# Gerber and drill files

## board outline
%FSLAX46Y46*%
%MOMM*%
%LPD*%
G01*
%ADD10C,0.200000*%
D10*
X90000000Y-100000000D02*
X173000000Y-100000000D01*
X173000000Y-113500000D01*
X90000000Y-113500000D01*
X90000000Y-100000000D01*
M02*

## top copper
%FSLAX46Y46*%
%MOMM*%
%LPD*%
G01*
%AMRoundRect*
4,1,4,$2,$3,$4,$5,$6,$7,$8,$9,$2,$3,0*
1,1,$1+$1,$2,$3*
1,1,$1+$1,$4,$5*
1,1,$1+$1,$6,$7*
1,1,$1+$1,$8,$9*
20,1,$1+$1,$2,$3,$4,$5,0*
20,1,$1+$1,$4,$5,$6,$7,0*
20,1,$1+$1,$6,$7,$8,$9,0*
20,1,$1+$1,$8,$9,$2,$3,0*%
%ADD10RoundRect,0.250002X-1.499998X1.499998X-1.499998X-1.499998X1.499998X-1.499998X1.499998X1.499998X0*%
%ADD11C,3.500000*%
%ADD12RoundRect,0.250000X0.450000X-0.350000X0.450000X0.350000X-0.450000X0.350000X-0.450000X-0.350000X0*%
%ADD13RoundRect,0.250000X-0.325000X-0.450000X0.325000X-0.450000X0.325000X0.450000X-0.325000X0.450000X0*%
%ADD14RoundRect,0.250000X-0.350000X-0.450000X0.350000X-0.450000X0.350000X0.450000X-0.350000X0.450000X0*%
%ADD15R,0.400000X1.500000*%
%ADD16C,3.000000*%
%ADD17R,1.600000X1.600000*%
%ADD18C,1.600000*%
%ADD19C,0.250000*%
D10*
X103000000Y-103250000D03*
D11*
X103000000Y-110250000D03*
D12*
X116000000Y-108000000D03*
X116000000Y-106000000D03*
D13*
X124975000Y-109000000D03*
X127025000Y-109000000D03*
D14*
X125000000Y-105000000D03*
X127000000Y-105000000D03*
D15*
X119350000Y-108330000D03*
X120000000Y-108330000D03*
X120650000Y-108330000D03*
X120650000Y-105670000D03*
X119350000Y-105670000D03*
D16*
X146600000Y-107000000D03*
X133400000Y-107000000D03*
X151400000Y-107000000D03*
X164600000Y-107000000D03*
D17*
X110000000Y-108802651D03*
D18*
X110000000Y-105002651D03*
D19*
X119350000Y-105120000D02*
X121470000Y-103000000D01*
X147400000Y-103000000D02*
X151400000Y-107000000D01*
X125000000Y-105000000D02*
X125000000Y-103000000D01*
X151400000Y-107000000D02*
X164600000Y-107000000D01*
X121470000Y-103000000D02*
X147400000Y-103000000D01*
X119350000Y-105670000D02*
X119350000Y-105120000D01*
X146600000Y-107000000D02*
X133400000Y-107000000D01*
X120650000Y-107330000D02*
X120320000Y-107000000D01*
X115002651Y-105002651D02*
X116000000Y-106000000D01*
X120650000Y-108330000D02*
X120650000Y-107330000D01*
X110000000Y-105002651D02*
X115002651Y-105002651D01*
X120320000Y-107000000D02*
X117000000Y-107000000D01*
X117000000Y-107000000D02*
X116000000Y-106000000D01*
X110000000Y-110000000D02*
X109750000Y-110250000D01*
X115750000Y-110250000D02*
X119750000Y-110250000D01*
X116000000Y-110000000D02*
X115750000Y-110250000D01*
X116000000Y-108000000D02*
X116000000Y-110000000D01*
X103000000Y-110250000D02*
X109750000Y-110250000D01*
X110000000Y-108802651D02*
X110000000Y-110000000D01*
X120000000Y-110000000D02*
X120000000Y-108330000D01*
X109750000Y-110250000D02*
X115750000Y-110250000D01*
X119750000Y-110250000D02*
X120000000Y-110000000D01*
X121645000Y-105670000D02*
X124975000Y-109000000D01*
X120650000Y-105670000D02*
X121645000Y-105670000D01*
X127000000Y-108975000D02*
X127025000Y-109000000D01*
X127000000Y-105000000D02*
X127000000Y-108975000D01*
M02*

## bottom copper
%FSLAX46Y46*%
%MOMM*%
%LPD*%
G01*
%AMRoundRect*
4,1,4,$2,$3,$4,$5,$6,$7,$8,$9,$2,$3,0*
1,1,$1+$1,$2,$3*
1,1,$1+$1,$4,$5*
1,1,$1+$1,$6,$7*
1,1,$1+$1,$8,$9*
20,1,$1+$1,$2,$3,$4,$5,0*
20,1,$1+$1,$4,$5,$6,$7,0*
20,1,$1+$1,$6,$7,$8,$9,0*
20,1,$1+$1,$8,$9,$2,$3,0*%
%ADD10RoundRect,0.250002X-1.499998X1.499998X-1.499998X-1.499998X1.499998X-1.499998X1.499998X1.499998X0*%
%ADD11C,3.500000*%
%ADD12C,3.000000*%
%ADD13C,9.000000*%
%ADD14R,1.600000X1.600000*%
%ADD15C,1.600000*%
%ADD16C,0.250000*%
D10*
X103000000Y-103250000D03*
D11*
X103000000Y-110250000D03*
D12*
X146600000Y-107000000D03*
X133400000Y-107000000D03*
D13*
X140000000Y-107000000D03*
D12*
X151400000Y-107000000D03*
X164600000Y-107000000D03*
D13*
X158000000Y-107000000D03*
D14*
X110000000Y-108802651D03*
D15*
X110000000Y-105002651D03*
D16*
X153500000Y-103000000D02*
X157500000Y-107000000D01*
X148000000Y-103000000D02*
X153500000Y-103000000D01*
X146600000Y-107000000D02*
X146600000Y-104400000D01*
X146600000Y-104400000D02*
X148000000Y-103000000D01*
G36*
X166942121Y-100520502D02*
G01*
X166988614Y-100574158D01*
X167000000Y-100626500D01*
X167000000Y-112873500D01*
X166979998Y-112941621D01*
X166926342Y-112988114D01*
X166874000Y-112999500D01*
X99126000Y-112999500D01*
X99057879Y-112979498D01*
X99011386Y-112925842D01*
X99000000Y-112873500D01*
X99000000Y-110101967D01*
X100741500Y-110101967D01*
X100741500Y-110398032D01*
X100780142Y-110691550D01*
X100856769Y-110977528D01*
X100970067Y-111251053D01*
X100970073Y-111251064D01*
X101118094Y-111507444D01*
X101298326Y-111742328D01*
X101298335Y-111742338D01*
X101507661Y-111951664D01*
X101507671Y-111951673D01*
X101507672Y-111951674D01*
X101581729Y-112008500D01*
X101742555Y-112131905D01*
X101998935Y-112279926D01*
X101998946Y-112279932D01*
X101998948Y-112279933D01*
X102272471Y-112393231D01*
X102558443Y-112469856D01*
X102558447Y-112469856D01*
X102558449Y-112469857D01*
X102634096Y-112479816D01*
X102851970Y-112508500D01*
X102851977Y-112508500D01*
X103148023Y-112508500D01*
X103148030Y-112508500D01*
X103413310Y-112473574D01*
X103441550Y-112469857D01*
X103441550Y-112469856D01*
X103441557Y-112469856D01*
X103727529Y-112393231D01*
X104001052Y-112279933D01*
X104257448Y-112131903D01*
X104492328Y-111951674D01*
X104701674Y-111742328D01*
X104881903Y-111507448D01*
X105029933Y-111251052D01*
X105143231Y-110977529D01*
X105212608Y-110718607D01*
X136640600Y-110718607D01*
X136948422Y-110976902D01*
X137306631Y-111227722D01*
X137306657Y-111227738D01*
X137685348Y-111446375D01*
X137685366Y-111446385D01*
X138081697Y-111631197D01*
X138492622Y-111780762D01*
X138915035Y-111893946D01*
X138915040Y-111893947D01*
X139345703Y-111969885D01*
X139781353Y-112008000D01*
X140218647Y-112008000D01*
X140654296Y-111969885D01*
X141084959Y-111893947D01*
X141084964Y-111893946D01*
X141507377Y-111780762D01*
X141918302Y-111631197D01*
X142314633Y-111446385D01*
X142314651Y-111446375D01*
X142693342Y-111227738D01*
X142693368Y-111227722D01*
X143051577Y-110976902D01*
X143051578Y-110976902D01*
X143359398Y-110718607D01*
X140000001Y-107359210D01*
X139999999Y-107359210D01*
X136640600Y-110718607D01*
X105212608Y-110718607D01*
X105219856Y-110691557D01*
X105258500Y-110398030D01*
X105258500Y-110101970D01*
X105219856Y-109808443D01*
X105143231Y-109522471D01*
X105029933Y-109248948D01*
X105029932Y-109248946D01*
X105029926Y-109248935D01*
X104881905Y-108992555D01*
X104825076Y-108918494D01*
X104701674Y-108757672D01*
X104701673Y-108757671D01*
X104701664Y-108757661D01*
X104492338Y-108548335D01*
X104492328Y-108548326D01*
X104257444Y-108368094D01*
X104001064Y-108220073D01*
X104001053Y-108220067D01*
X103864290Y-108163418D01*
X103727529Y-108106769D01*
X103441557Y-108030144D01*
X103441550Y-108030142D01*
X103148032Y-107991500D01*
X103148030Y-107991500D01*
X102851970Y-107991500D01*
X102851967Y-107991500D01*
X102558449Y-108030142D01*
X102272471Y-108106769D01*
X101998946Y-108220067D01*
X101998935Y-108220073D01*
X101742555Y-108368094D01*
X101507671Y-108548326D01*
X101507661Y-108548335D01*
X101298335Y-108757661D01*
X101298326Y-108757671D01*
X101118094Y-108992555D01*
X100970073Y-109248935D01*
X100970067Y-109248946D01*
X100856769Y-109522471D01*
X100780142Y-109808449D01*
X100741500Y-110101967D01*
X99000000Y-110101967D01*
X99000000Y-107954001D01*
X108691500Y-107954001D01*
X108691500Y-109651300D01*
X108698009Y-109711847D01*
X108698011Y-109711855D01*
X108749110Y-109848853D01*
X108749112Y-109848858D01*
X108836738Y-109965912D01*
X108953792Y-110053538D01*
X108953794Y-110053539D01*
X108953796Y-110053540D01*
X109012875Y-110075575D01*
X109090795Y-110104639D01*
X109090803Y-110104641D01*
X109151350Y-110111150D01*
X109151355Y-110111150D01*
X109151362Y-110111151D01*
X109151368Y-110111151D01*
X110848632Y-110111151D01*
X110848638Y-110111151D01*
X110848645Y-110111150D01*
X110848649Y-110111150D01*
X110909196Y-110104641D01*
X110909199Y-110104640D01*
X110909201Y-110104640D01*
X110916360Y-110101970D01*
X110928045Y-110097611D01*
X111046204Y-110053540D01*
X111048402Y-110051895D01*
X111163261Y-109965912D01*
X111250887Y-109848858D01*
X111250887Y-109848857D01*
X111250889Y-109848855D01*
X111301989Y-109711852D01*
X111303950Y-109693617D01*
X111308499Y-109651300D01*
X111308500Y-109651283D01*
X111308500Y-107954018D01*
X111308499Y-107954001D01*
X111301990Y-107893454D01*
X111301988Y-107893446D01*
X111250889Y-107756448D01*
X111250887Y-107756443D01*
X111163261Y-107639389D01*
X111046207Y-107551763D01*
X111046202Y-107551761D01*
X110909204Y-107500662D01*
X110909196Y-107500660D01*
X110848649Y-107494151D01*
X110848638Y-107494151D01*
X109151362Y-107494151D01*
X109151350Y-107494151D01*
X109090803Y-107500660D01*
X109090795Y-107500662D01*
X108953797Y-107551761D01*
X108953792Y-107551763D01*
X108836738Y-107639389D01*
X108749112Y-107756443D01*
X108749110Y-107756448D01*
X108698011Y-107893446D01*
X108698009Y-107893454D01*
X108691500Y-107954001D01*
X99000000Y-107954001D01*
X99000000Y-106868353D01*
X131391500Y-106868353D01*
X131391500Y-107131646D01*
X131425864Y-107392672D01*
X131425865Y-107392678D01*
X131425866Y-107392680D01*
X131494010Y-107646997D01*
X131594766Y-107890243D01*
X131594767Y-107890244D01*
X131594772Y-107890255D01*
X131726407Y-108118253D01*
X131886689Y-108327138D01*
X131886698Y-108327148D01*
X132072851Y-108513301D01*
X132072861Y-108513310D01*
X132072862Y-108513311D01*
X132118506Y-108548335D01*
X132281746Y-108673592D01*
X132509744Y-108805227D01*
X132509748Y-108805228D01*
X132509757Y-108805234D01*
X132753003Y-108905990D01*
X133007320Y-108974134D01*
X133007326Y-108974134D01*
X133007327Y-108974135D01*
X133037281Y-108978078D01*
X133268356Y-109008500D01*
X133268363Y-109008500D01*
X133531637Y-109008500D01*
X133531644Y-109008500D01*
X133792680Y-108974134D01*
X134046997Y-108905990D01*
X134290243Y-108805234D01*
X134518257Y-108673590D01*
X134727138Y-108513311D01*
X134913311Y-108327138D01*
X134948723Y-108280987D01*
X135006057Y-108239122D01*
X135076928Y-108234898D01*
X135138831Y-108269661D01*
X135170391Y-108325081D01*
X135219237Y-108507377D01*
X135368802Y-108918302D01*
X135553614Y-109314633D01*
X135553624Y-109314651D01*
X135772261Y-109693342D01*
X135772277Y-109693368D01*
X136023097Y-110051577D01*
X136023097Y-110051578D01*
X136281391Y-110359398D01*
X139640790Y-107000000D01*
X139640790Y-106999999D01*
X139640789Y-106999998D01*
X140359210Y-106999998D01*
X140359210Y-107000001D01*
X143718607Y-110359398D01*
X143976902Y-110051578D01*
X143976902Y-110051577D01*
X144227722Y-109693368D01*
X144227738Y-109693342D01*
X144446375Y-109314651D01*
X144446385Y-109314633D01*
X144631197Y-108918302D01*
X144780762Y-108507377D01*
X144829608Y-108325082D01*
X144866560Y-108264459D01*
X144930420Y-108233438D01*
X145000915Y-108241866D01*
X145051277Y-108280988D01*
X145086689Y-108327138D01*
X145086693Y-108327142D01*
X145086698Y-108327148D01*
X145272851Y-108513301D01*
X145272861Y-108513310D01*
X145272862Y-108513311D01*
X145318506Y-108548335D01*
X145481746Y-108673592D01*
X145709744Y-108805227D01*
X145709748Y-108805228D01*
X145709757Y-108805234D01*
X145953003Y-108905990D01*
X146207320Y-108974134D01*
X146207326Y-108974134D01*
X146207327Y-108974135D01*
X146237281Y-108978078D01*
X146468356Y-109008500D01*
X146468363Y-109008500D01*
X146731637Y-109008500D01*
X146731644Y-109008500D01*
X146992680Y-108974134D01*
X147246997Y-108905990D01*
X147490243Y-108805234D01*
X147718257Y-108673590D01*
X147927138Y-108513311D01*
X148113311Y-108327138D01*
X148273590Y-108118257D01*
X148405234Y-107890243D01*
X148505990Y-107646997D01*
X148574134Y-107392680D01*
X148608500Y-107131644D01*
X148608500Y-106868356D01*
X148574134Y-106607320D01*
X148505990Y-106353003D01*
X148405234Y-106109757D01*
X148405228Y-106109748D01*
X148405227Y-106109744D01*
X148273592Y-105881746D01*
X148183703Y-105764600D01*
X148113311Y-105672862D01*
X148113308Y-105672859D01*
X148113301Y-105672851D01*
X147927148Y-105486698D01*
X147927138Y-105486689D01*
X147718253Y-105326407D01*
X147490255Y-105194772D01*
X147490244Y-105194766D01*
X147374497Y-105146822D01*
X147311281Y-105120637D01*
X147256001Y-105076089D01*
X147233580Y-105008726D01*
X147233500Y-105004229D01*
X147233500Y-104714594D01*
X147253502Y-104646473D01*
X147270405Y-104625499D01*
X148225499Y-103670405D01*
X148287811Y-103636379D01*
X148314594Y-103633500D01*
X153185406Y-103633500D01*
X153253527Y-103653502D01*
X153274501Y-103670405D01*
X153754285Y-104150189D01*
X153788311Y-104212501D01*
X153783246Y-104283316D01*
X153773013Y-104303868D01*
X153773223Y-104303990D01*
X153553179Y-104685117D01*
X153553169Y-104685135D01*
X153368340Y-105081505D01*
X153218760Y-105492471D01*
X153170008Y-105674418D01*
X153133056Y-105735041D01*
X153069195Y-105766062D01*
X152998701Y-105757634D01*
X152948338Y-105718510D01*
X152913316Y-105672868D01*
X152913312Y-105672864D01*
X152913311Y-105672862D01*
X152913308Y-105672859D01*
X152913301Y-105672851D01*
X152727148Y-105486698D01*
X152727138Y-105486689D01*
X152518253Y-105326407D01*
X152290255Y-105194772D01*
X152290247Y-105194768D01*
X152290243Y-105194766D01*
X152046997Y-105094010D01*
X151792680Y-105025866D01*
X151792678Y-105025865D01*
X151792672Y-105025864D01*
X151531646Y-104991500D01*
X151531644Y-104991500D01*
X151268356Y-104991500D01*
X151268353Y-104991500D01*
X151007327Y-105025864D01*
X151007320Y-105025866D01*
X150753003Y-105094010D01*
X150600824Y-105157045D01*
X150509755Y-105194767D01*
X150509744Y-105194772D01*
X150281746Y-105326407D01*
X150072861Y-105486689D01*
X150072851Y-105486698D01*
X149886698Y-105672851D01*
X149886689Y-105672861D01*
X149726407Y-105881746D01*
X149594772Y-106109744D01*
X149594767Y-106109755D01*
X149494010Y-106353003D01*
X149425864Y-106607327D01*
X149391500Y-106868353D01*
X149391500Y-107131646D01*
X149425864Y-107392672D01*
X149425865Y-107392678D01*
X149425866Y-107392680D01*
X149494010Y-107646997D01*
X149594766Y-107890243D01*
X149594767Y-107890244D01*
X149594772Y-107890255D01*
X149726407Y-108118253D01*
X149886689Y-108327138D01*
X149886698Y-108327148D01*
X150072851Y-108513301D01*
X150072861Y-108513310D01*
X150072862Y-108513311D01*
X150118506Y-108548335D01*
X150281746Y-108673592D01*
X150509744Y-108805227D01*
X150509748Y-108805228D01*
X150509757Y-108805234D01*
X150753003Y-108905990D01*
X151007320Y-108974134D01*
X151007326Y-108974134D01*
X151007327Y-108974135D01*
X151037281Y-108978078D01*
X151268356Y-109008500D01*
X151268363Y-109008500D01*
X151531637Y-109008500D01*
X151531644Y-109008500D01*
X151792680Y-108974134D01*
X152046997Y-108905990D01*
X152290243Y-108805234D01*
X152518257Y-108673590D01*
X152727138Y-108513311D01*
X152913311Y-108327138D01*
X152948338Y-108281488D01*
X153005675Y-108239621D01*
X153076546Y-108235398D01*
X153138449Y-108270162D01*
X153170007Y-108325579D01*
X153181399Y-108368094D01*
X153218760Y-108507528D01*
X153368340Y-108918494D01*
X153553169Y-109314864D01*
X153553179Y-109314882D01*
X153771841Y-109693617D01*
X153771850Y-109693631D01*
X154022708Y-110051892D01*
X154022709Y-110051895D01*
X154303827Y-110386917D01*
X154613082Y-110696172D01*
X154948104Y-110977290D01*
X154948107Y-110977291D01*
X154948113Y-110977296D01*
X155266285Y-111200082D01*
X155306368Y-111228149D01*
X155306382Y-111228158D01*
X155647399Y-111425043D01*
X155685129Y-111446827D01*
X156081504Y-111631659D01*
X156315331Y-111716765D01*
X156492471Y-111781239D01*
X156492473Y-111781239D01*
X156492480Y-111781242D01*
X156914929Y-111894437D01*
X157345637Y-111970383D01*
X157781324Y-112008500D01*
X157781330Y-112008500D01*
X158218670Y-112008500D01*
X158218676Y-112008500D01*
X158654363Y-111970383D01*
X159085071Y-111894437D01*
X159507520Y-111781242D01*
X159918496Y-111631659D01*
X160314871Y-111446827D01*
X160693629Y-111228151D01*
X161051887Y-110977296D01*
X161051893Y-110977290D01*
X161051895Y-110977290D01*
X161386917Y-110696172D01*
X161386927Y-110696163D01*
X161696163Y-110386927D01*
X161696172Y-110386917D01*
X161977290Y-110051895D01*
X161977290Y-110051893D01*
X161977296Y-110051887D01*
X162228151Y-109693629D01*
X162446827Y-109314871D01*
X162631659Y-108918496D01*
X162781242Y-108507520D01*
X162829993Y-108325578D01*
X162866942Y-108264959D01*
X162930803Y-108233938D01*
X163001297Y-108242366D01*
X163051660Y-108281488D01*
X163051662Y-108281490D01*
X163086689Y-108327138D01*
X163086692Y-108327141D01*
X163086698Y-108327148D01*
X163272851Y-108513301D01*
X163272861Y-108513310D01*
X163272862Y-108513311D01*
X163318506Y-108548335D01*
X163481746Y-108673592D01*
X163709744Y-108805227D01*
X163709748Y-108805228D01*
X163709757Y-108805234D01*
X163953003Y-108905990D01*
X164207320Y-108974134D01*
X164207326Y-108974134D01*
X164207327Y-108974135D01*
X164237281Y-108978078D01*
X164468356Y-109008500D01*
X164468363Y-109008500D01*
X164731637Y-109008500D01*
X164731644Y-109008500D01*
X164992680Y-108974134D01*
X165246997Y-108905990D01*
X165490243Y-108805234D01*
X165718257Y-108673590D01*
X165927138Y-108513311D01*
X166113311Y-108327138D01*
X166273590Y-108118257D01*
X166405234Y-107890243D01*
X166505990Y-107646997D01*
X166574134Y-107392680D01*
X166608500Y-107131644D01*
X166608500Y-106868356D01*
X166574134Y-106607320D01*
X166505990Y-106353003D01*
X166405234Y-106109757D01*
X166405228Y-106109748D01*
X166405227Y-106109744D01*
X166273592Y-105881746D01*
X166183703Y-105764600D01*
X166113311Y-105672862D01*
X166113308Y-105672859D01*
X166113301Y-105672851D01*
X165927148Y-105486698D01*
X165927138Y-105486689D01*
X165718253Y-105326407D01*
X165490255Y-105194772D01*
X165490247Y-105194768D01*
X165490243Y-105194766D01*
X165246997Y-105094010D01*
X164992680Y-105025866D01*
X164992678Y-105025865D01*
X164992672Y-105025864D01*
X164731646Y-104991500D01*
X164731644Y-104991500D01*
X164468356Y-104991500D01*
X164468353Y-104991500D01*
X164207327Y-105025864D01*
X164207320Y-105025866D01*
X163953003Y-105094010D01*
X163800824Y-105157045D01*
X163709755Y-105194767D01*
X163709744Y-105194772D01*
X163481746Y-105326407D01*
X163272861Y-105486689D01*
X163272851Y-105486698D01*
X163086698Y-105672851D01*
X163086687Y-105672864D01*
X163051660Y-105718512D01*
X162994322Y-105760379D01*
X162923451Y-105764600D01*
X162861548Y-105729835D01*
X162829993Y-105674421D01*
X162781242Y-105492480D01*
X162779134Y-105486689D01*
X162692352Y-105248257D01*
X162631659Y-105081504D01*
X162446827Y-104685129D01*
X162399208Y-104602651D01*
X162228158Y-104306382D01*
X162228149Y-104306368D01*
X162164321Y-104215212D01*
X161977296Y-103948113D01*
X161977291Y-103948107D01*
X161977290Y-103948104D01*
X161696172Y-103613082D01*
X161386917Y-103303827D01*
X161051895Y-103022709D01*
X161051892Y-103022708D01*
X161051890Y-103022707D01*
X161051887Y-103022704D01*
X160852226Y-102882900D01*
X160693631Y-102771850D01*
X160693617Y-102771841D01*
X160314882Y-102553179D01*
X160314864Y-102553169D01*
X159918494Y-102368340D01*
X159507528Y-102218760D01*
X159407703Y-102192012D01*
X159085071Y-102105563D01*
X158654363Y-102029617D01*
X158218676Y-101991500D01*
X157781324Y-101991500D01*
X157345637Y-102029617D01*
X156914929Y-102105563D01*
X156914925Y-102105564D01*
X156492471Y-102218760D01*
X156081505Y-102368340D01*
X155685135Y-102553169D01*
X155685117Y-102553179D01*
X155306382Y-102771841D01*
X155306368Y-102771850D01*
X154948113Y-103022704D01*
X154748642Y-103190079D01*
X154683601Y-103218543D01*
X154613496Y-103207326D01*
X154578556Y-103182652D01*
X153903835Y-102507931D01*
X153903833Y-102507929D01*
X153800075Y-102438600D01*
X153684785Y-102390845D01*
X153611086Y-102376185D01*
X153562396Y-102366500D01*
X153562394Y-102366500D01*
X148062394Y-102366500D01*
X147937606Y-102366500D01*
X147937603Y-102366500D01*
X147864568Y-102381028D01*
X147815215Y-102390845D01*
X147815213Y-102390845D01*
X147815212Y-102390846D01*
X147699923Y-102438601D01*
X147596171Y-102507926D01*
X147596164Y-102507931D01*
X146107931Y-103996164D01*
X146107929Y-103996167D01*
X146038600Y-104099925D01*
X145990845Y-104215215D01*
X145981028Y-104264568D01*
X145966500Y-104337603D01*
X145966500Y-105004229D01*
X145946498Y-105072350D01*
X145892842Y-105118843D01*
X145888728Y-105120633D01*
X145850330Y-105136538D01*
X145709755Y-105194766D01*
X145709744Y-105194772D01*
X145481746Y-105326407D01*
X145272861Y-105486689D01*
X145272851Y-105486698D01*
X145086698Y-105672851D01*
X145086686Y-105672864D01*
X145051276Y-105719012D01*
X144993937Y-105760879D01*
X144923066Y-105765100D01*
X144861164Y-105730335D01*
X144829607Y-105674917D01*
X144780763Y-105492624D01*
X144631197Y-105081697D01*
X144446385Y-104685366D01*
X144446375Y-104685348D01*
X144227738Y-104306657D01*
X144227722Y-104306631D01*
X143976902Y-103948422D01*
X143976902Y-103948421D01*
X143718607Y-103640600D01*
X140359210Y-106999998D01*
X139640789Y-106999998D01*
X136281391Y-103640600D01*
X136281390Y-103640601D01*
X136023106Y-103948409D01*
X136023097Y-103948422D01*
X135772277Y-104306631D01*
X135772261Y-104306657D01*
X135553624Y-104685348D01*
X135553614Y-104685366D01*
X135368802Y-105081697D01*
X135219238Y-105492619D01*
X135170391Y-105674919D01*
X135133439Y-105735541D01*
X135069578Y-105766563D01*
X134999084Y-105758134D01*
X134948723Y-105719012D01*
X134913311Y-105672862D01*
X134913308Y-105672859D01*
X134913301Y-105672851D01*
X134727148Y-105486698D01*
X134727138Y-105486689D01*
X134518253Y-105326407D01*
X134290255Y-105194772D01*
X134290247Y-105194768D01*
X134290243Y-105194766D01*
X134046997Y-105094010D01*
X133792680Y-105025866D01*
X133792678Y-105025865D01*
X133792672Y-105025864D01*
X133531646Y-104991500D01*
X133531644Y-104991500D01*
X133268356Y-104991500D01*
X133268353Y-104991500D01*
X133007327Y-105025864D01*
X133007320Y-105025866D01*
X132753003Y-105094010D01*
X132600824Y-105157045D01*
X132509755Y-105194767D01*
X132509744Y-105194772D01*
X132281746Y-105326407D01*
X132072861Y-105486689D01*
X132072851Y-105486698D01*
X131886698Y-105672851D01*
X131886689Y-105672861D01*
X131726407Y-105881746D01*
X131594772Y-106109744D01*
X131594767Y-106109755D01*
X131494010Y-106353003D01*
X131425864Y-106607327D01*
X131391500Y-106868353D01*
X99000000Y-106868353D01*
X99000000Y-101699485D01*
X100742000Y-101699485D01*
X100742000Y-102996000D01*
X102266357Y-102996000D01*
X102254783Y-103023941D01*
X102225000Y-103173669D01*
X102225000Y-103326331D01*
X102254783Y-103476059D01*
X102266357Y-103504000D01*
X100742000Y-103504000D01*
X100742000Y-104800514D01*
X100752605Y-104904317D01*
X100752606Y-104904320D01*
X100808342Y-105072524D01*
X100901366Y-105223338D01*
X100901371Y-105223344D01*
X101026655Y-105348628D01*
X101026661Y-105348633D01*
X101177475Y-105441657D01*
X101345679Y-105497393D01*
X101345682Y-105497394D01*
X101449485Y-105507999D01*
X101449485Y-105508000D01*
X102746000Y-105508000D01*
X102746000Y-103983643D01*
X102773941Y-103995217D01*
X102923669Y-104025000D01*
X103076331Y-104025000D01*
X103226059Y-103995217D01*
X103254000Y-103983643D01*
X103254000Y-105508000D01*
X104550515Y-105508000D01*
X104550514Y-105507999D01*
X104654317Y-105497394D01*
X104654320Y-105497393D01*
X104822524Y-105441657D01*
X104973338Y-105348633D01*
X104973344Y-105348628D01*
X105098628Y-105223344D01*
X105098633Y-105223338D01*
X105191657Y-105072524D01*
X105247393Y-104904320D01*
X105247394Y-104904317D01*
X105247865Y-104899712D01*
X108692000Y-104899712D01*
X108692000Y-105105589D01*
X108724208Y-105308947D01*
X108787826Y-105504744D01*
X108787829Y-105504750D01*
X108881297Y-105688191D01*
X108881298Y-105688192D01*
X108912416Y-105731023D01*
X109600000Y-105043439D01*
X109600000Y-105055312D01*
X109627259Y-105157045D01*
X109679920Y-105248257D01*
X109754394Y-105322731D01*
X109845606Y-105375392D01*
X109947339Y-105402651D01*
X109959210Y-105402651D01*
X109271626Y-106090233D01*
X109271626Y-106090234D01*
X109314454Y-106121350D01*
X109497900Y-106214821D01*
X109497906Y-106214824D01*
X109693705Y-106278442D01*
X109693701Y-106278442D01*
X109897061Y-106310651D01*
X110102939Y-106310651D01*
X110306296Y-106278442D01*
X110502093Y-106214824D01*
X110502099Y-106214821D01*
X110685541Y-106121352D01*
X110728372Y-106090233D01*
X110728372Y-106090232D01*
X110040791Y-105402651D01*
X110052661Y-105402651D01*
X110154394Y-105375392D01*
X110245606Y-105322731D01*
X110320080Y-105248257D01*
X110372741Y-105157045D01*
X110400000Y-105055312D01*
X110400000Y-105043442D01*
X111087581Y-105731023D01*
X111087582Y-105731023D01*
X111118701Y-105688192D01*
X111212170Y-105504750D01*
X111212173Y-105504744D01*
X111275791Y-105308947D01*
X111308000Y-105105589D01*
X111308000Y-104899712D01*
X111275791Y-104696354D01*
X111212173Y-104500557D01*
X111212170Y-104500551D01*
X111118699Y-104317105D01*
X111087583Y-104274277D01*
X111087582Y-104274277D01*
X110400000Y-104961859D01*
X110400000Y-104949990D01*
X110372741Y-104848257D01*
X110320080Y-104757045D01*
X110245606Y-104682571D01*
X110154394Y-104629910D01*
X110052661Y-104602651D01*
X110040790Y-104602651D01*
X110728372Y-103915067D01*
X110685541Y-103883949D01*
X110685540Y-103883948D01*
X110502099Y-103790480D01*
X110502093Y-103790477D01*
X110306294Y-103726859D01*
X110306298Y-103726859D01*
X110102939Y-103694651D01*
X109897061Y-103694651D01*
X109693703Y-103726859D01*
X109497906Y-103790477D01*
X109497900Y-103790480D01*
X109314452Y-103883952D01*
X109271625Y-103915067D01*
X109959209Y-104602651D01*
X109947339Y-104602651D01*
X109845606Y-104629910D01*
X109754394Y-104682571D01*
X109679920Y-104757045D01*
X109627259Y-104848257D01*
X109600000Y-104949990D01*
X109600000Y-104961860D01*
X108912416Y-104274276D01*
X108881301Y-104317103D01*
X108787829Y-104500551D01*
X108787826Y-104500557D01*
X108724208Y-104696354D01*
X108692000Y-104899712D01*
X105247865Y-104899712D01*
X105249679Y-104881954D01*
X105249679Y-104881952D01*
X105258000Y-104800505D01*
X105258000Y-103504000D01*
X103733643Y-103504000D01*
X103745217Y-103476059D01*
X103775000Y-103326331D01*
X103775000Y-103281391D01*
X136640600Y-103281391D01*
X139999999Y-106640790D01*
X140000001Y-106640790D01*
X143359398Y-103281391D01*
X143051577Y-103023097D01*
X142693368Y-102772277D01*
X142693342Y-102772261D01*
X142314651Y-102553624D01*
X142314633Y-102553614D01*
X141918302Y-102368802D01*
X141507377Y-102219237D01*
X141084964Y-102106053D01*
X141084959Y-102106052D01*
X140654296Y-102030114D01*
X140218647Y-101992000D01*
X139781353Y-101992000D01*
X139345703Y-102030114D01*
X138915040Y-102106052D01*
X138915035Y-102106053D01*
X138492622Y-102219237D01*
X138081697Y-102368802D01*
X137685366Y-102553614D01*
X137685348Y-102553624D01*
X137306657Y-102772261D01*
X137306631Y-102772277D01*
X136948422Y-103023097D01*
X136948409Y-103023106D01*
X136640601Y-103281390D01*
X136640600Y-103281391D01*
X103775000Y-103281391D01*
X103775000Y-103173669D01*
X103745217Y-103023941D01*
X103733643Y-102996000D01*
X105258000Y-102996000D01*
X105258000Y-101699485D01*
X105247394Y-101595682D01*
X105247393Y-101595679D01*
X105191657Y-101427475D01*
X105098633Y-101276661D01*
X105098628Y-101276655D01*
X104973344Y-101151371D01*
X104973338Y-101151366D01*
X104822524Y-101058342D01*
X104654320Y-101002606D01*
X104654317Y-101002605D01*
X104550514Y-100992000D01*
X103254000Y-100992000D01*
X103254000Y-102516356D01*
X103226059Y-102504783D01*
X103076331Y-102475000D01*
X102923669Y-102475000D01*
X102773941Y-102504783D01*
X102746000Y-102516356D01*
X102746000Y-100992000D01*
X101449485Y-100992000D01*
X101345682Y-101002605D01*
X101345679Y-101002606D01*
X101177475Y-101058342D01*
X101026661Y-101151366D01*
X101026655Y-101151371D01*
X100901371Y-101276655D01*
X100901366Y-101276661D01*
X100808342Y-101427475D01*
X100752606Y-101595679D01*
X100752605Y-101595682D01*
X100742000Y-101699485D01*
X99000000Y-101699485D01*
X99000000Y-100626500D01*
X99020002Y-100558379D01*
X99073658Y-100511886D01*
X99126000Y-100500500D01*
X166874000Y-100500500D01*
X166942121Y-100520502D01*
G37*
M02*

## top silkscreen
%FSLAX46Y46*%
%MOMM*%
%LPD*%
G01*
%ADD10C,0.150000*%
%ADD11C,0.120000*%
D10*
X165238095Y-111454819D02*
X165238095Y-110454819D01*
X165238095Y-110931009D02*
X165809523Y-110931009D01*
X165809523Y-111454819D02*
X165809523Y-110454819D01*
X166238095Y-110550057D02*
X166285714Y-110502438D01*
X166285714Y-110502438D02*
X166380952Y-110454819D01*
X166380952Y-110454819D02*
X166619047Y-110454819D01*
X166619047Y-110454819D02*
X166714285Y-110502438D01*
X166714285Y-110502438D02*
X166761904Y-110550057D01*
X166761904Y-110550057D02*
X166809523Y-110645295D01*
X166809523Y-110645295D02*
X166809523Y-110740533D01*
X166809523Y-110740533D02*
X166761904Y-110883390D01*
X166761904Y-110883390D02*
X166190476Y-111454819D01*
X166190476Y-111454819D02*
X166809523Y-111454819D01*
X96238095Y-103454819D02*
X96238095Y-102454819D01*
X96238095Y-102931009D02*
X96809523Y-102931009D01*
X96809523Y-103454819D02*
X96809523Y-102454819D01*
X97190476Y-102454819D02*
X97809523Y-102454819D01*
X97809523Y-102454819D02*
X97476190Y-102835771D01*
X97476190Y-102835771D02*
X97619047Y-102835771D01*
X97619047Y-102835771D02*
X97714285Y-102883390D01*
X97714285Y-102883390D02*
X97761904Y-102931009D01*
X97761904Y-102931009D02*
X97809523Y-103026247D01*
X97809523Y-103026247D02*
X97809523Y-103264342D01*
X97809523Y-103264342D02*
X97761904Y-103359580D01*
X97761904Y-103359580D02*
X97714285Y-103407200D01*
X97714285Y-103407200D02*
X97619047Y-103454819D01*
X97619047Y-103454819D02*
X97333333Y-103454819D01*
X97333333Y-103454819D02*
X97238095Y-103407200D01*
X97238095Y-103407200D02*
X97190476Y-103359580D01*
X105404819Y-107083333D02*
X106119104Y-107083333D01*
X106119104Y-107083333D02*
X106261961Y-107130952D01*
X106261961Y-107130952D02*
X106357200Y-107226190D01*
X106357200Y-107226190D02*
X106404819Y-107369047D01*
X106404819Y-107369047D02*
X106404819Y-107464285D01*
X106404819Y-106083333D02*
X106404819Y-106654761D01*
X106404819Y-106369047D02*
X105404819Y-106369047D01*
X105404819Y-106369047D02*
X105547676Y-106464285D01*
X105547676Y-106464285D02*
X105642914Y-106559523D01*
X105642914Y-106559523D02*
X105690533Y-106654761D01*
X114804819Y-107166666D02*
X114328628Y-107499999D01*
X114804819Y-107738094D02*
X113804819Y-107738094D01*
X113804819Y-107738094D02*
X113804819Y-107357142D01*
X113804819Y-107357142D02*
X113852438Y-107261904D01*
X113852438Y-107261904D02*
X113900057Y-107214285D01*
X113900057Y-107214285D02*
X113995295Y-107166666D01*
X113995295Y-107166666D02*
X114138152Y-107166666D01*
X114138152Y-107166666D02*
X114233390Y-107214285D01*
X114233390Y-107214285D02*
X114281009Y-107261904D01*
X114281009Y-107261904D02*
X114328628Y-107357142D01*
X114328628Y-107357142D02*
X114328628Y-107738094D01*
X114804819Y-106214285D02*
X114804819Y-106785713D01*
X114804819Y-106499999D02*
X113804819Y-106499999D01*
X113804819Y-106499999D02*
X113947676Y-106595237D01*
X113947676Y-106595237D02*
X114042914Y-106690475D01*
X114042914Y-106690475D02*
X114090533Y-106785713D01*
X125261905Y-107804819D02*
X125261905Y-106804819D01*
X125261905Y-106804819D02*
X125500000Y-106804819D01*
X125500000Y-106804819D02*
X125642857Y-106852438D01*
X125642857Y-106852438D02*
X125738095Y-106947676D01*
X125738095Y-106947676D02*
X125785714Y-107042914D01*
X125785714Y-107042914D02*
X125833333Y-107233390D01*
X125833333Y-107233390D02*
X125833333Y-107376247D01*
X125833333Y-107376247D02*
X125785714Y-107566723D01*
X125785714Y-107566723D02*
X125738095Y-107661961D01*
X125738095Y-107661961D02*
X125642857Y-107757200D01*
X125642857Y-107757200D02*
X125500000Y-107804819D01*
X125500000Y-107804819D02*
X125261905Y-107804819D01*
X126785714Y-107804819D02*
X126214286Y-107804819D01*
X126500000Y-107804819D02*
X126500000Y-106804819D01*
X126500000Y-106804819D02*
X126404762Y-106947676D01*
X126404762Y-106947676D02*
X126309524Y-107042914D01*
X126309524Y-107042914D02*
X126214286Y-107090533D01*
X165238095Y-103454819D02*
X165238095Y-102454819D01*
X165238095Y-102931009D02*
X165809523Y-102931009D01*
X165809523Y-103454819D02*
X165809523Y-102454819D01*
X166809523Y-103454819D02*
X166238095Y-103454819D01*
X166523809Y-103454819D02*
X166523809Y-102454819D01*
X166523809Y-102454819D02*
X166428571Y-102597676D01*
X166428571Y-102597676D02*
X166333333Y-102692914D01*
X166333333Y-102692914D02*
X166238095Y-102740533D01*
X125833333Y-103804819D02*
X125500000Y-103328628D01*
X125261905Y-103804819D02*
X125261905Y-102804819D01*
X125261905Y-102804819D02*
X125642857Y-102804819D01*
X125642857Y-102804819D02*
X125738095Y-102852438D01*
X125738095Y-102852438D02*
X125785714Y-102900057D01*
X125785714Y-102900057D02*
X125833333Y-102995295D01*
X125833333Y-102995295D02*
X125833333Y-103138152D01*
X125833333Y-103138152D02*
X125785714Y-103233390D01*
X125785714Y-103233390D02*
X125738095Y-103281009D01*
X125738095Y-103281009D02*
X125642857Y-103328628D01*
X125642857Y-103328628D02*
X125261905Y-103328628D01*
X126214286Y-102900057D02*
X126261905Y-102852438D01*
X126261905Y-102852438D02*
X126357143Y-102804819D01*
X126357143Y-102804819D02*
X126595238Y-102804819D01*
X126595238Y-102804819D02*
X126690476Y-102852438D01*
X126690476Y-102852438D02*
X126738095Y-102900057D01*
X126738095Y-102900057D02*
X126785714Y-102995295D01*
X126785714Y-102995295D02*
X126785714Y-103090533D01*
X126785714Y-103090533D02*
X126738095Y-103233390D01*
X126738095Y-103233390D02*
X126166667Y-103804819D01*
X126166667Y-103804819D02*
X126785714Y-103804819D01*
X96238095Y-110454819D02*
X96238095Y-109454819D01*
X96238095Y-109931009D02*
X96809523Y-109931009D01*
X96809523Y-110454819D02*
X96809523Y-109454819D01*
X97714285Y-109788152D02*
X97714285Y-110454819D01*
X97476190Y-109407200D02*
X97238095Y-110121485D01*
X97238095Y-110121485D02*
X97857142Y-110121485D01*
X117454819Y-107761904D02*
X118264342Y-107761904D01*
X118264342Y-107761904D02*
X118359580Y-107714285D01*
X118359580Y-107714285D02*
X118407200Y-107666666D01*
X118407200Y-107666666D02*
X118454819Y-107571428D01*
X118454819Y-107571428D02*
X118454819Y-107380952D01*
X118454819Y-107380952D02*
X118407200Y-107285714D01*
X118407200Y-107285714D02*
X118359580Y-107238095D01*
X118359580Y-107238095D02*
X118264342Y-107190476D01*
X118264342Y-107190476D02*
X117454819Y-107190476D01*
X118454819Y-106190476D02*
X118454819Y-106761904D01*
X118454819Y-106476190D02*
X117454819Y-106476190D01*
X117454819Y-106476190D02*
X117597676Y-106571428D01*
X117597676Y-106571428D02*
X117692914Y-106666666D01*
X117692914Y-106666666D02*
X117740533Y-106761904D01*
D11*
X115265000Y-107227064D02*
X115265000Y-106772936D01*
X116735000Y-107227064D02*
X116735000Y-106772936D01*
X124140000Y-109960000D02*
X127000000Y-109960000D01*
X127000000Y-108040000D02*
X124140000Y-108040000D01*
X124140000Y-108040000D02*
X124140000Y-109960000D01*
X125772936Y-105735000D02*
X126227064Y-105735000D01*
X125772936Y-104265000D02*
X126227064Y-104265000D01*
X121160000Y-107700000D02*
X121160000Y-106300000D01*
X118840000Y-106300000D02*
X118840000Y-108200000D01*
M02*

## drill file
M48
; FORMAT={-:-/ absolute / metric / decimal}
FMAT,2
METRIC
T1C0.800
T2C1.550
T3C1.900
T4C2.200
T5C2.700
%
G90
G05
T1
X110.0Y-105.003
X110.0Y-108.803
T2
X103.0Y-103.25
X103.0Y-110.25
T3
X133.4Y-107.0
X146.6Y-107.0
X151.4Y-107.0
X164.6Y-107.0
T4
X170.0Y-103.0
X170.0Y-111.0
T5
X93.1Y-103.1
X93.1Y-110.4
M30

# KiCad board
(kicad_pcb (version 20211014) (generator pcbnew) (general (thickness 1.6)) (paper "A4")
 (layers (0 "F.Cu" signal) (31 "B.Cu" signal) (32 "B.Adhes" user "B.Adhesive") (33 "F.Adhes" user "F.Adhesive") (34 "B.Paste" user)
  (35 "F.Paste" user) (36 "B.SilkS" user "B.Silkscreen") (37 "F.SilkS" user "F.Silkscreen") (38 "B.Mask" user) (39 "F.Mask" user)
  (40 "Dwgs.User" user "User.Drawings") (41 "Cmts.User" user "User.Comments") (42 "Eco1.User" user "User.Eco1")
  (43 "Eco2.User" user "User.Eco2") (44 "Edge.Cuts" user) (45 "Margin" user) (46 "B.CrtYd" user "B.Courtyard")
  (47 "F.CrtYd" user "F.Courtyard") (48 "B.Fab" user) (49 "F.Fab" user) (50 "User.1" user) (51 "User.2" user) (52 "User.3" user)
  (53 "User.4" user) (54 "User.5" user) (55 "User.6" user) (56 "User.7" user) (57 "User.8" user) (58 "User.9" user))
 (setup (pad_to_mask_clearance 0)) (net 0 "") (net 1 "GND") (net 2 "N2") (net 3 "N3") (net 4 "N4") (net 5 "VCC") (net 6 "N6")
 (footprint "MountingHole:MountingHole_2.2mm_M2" (layer "F.Cu") (at 170 111)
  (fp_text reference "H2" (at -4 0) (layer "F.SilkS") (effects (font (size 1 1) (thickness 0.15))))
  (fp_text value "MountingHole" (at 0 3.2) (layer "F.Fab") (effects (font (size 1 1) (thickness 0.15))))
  (pad "" np_thru_hole circle (at 0 0) (size 2.2 2.2) (drill 2.2) (layers *.Cu *.Mask)))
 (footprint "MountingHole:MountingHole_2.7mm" (layer "F.Cu") (at 93.1 103.1)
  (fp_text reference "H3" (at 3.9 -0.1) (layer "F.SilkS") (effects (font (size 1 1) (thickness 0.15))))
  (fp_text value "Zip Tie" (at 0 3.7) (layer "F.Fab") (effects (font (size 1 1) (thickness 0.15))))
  (pad "" np_thru_hole circle (at 0 0) (size 2.7 2.7) (drill 2.7) (layers *.Cu *.Mask)))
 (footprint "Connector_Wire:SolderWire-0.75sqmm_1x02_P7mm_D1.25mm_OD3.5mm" (layer "F.Cu") (at 103 103.25 -90)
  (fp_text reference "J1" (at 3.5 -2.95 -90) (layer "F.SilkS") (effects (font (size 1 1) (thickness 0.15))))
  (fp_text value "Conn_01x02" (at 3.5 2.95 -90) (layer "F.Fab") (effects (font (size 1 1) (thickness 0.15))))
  (pad "1" thru_hole roundrect (at 0 0 270) (size 3.5 3.5) (drill 1.55) (layers *.Cu *.Mask) (roundrect_rratio 0.07142914286) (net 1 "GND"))
  (pad "2" thru_hole circle (at 7 0 270) (size 3.5 3.5) (drill 1.55) (layers *.Cu *.Mask) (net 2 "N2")))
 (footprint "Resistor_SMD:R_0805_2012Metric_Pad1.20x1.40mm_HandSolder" (layer "F.Cu") (at 116 107 90)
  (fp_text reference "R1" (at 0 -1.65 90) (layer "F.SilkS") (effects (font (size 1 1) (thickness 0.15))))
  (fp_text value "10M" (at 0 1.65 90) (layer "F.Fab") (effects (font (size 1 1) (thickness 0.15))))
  (fp_line (start -0.227064 -0.735) (end 0.227064 -0.735) (layer "F.SilkS") (width 0.12))
  (fp_line (start -0.227064 0.735) (end 0.227064 0.735) (layer "F.SilkS") (width 0.12))
  (pad "1" smd roundrect (at -1 0 90) (size 1.2 1.4) (layers "F.Cu" "F.Paste" "F.Mask") (roundrect_rratio 0.2083333333) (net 2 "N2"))
  (pad "2" smd roundrect (at 1 0 90) (size 1.2 1.4) (layers "F.Cu" "F.Paste" "F.Mask") (roundrect_rratio 0.2083333333) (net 1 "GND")))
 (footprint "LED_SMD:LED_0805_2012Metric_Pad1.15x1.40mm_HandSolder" (layer "F.Cu") (at 126 109)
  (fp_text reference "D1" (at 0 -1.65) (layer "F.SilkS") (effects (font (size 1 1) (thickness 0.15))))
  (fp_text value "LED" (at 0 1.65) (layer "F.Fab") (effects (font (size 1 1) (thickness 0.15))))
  (fp_line (start -1.86 0.96) (end 1 0.96) (layer "F.SilkS") (width 0.12))
  (fp_line (start 1 -0.96) (end -1.86 -0.96) (layer "F.SilkS") (width 0.12))
  (fp_line (start -1.86 -0.96) (end -1.86 0.96) (layer "F.SilkS") (width 0.12))
  (pad "1" smd roundrect (at -1.025 0) (size 1.15 1.4) (layers "F.Cu" "F.Paste" "F.Mask") (roundrect_rratio 0.2173913043) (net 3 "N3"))
  (pad "2" smd roundrect (at 1.025 0) (size 1.15 1.4) (layers "F.Cu" "F.Paste" "F.Mask") (roundrect_rratio 0.2173913043) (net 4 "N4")))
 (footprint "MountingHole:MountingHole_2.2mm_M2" (layer "F.Cu") (at 170 103)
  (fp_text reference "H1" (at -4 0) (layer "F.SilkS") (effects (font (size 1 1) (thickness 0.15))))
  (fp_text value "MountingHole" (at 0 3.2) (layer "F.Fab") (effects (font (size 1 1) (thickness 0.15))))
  (pad "" np_thru_hole circle (at 0 0) (size 2.2 2.2) (drill 2.2) (layers *.Cu *.Mask)))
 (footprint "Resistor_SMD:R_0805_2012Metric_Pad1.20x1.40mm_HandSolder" (layer "F.Cu") (at 126 105)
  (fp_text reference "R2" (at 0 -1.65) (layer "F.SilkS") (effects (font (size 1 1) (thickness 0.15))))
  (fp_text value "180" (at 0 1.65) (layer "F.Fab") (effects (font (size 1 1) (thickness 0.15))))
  (fp_line (start -0.227064 0.735) (end 0.227064 0.735) (layer "F.SilkS") (width 0.12))
  (fp_line (start -0.227064 -0.735) (end 0.227064 -0.735) (layer "F.SilkS") (width 0.12))
  (pad "1" smd roundrect (at -1 0) (size 1.2 1.4) (layers "F.Cu" "F.Paste" "F.Mask") (roundrect_rratio 0.2083333333) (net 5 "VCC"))
  (pad "2" smd roundrect (at 1 0) (size 1.2 1.4) (layers "F.Cu" "F.Paste" "F.Mask") (roundrect_rratio 0.2083333333) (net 4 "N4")))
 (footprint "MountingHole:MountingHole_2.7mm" (layer "F.Cu") (at 93.1 110.4)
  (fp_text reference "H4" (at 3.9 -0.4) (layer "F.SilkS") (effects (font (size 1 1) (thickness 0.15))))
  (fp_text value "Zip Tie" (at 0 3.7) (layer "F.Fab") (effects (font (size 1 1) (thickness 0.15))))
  (pad "" np_thru_hole circle (at 0 0) (size 2.7 2.7) (drill 2.7) (layers *.Cu *.Mask)))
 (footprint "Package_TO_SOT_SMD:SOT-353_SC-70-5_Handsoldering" (layer "F.Cu") (at 120 107 90)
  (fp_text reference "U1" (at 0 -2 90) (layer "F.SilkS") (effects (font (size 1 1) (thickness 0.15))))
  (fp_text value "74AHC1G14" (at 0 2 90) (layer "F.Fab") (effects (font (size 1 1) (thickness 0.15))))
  (fp_line (start -0.7 1.16) (end 0.7 1.16) (layer "F.SilkS") (width 0.12))
  (fp_line (start 0.7 -1.16) (end -1.2 -1.16) (layer "F.SilkS") (width 0.12))
  (pad "1" smd rect (at -1.33 -0.65 90) (size 1.5 0.4) (layers "F.Cu" "F.Paste" "F.Mask"))
  (pad "2" smd rect (at -1.33 0 90) (size 1.5 0.4) (layers "F.Cu" "F.Paste" "F.Mask") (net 2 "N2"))
  (pad "3" smd rect (at -1.33 0.65 90) (size 1.5 0.4) (layers "F.Cu" "F.Paste" "F.Mask") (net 1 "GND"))
  (pad "4" smd rect (at 1.33 0.65 90) (size 1.5 0.4) (layers "F.Cu" "F.Paste" "F.Mask") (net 3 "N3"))
  (pad "5" smd rect (at 1.33 -0.65 90) (size 1.5 0.4) (layers "F.Cu" "F.Paste" "F.Mask") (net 5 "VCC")))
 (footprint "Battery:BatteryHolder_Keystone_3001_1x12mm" (layer "B.Cu") (at 140 107 180)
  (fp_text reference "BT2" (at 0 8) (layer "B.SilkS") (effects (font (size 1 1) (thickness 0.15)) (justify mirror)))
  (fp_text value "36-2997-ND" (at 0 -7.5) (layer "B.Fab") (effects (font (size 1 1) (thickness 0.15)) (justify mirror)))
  (pad "1" thru_hole circle (at -6.6 0 180) (size 3 3) (drill 1.9) (layers *.Cu *.Mask) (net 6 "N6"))
  (pad "1" thru_hole circle (at 6.6 0 180) (size 3 3) (drill 1.9) (layers *.Cu *.Mask) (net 6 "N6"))
  (pad "2" smd circle (at 0 0 180) (size 9 9) (layers "B.Cu" "B.Mask") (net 1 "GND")))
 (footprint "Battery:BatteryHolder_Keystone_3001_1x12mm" (layer "B.Cu") (at 158 107 180)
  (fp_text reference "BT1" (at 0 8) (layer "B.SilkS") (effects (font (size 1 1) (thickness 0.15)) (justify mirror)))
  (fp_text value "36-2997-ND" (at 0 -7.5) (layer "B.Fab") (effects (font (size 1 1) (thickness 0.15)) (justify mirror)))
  (pad "1" thru_hole circle (at 6.6 0 180) (size 3 3) (drill 1.9) (layers *.Cu *.Mask) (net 5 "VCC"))
  (pad "1" thru_hole circle (at -6.6 0 180) (size 3 3) (drill 1.9) (layers *.Cu *.Mask) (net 5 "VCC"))
  (pad "2" smd circle (at 0 0 180) (size 9 9) (layers "B.Cu" "B.Mask") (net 6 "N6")))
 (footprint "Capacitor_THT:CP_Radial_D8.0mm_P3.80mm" (layer "B.Cu") (at 110 108.802651 90)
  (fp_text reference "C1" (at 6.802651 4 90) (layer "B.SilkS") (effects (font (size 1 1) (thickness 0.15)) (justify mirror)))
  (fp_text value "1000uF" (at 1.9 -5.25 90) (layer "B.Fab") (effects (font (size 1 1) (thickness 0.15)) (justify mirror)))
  (pad "1" thru_hole rect (at 0 0 90) (size 1.6 1.6) (drill 0.8) (layers *.Cu *.Mask) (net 2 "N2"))
  (pad "2" thru_hole circle (at 3.8 0 90) (size 1.6 1.6) (drill 0.8) (layers *.Cu *.Mask) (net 1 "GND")))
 (gr_rect (start 90 100) (end 173 113.5) (layer "Edge.Cuts") (width 0.2) (fill none))
 (segment (start 119.35 105.12) (end 121.47 103) (width 0.25) (layer "F.Cu") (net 5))
 (segment (start 147.4 103) (end 151.4 107) (width 0.25) (layer "F.Cu") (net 5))
 (segment (start 125 105) (end 125 103) (width 0.25) (layer "F.Cu") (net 5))
 (segment (start 151.4 107) (end 164.6 107) (width 0.25) (layer "F.Cu") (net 5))
 (segment (start 121.47 103) (end 147.4 103) (width 0.25) (layer "F.Cu") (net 5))
 (segment (start 119.35 105.67) (end 119.35 105.12) (width 0.25) (layer "F.Cu") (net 5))
 (segment (start 146.6 107) (end 133.4 107) (width 0.25) (layer "F.Cu") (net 6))
 (segment (start 153.5 103) (end 157.5 107) (width 0.25) (layer "B.Cu") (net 6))
 (segment (start 148 103) (end 153.5 103) (width 0.25) (layer "B.Cu") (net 6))
 (segment (start 146.6 107) (end 146.6 104.4) (width 0.25) (layer "B.Cu") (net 6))
 (segment (start 146.6 104.4) (end 148 103) (width 0.25) (layer "B.Cu") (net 6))
 (segment (start 120.65 107.33) (end 120.32 107) (width 0.25) (layer "F.Cu") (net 1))
 (segment (start 115.002651 105.002651) (end 116 106) (width 0.25) (layer "F.Cu") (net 1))
 (segment (start 120.65 108.33) (end 120.65 107.33) (width 0.25) (layer "F.Cu") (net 1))
 (segment (start 110 105.002651) (end 115.002651 105.002651) (width 0.25) (layer "F.Cu") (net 1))
 (segment (start 120.32 107) (end 117 107) (width 0.25) (layer "F.Cu") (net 1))
 (segment (start 117 107) (end 116 106) (width 0.25) (layer "F.Cu") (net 1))
 (segment (start 110 110) (end 109.75 110.25) (width 0.25) (layer "F.Cu") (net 2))
 (segment (start 115.75 110.25) (end 119.75 110.25) (width 0.25) (layer "F.Cu") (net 2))
 (segment (start 116 110) (end 115.75 110.25) (width 0.25) (layer "F.Cu") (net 2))
 (segment (start 116 108) (end 116 110) (width 0.25) (layer "F.Cu") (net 2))
 (segment (start 103 110.25) (end 109.75 110.25) (width 0.25) (layer "F.Cu") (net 2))
 (segment (start 110 108.802651) (end 110 110) (width 0.25) (layer "F.Cu") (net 2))
 (segment (start 120 110) (end 120 108.33) (width 0.25) (layer "F.Cu") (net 2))
 (segment (start 109.75 110.25) (end 115.75 110.25) (width 0.25) (layer "F.Cu") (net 2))
 (segment (start 119.75 110.25) (end 120 110) (width 0.25) (layer "F.Cu") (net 2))
 (segment (start 121.645 105.67) (end 124.975 109) (width 0.25) (layer "F.Cu") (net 3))
 (segment (start 120.65 105.67) (end 121.645 105.67) (width 0.25) (layer "F.Cu") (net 3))
 (segment (start 127 108.975) (end 127.025 109) (width 0.25) (layer "F.Cu") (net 4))
 (segment (start 127 105) (end 127 108.975) (width 0.25) (layer "F.Cu") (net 4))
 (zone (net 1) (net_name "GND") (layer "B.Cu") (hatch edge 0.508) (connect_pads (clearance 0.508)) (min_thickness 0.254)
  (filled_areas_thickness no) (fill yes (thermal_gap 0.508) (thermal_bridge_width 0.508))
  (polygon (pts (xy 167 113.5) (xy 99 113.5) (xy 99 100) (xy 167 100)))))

